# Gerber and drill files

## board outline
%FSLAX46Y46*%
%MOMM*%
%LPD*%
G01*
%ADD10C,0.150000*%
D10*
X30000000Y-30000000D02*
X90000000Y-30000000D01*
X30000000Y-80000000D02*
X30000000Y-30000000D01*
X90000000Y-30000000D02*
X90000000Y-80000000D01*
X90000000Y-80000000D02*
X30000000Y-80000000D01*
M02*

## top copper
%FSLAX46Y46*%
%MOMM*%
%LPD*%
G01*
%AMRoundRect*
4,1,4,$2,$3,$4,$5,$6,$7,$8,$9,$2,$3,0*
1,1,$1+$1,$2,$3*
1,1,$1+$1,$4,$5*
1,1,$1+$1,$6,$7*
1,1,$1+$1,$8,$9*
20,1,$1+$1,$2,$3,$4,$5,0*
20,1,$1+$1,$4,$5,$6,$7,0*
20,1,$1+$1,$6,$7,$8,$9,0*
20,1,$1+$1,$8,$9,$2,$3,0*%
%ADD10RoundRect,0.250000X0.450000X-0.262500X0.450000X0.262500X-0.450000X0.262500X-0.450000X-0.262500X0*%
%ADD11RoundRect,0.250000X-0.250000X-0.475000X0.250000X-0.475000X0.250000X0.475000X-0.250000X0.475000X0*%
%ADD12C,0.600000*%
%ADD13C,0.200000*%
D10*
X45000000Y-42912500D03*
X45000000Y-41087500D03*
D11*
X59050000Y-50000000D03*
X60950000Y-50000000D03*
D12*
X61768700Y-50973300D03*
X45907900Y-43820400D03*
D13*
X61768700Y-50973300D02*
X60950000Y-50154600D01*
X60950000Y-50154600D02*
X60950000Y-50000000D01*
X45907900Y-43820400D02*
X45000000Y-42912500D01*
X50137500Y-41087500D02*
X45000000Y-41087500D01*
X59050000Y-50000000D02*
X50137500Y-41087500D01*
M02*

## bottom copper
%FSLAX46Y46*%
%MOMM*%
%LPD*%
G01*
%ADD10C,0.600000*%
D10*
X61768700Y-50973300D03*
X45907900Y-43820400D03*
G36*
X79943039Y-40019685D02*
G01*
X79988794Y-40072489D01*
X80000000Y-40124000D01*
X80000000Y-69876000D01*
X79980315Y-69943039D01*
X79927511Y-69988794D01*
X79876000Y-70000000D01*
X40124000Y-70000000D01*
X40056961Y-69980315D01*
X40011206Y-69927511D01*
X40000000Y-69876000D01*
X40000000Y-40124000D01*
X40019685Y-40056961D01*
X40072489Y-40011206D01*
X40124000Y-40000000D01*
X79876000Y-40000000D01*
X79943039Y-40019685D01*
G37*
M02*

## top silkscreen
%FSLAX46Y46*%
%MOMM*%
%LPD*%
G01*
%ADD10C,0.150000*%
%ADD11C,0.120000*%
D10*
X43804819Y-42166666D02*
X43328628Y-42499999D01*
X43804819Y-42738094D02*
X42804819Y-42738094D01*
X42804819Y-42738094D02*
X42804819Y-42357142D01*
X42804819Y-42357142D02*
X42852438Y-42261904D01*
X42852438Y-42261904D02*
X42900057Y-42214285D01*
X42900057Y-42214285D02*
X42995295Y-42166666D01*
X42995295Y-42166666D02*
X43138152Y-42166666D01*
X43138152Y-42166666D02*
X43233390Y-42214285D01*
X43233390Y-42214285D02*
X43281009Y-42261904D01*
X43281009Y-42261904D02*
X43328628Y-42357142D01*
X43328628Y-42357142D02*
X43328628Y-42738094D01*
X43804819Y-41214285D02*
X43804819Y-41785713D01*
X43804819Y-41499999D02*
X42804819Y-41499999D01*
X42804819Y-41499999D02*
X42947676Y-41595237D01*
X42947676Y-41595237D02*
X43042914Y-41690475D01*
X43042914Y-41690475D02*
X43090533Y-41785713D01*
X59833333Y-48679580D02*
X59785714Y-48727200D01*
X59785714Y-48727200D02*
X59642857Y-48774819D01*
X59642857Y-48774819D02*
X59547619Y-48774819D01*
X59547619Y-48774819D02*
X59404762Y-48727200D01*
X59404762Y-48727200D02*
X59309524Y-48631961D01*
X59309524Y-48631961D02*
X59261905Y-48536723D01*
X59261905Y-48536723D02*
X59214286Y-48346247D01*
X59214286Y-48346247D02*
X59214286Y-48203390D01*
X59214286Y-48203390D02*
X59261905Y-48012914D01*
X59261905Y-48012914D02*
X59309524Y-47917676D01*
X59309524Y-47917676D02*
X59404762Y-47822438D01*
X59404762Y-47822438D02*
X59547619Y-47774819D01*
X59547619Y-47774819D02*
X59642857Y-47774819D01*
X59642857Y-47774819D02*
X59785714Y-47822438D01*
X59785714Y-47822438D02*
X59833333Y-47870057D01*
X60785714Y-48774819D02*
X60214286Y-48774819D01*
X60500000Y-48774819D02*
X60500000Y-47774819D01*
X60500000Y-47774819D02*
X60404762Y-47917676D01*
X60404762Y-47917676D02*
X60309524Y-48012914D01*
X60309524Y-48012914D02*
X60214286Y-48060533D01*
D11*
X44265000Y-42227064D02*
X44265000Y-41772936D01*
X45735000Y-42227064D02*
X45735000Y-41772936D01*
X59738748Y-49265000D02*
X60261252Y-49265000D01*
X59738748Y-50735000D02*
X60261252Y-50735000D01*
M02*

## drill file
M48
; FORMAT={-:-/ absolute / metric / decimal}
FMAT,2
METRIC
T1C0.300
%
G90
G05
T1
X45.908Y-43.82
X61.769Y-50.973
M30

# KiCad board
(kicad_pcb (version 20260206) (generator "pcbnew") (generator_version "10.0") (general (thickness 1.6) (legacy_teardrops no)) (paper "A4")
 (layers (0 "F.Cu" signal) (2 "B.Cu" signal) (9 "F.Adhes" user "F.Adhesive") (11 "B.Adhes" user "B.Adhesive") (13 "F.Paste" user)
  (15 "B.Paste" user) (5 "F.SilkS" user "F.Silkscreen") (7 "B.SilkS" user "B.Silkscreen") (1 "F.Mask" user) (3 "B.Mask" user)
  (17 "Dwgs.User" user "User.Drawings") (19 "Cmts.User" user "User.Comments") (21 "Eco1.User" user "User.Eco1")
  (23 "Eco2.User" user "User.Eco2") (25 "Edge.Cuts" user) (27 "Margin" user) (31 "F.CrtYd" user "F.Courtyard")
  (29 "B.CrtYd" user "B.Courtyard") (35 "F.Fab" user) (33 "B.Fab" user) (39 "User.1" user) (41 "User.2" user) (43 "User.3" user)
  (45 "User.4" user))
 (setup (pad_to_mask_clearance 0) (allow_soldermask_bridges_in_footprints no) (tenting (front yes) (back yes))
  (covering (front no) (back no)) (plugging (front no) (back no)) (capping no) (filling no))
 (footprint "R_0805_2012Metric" (layer "F.Cu") (at 45 42 90)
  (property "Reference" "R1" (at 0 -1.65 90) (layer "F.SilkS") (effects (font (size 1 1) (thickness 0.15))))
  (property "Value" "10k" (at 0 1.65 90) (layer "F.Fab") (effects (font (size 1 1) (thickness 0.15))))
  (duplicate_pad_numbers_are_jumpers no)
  (fp_line (start -0.227064 -0.735) (end 0.227064 -0.735) (stroke (width 0.12) (type solid)) (layer "F.SilkS"))
  (fp_line (start -0.227064 0.735) (end 0.227064 0.735) (stroke (width 0.12) (type solid)) (layer "F.SilkS"))
  (pad "1" smd roundrect (at -0.9125 0 90) (size 1.025 1.4) (layers "F.Cu" "F.Mask" "F.Paste") (roundrect_rratio 0.243902) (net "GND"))
  (pad "2" smd roundrect (at 0.9125 0 90) (size 1.025 1.4) (layers "F.Cu" "F.Mask" "F.Paste") (roundrect_rratio 0.243902) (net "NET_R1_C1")))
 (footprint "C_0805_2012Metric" (layer "F.Cu") (at 60 50)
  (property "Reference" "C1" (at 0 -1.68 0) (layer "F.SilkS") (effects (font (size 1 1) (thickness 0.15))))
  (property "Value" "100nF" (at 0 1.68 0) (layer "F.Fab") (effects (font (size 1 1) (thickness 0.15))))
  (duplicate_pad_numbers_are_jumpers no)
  (fp_line (start -0.261252 -0.735) (end 0.261252 -0.735) (stroke (width 0.12) (type solid)) (layer "F.SilkS"))
  (fp_line (start -0.261252 0.735) (end 0.261252 0.735) (stroke (width 0.12) (type solid)) (layer "F.SilkS"))
  (pad "1" smd roundrect (at -0.95 0) (size 1 1.45) (layers "F.Cu" "F.Mask" "F.Paste") (roundrect_rratio 0.25) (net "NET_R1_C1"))
  (pad "2" smd roundrect (at 0.95 0) (size 1 1.45) (layers "F.Cu" "F.Mask" "F.Paste") (roundrect_rratio 0.25) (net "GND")))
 (gr_line (start 30 30) (end 90 30) (stroke (width 0.15) (type default)) (layer "Edge.Cuts"))
 (gr_line (start 30 80) (end 30 30) (stroke (width 0.15) (type default)) (layer "Edge.Cuts"))
 (gr_line (start 90 30) (end 90 80) (stroke (width 0.15) (type default)) (layer "Edge.Cuts"))
 (gr_line (start 90 80) (end 30 80) (stroke (width 0.15) (type default)) (layer "Edge.Cuts"))
 (segment (start 61.7687 50.9733) (end 60.95 50.1546) (width 0.2) (layer "F.Cu") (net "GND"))
 (segment (start 60.95 50.1546) (end 60.95 50) (width 0.2) (layer "F.Cu") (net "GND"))
 (segment (start 45.9079 43.8204) (end 45 42.9125) (width 0.2) (layer "F.Cu") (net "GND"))
 (via (at 61.7687 50.9733) (size 0.6) (drill 0.3) (layers "F.Cu" "B.Cu") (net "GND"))
 (via (at 45.9079 43.8204) (size 0.6) (drill 0.3) (layers "F.Cu" "B.Cu") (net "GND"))
 (segment (start 50.1375 41.0875) (end 45 41.0875) (width 0.2) (layer "F.Cu") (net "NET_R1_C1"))
 (segment (start 59.05 50) (end 50.1375 41.0875) (width 0.2) (layer "F.Cu") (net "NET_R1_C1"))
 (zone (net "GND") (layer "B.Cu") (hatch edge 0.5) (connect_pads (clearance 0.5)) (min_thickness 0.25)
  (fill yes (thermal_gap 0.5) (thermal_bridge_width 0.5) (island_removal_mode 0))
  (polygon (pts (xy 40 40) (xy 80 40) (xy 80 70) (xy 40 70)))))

